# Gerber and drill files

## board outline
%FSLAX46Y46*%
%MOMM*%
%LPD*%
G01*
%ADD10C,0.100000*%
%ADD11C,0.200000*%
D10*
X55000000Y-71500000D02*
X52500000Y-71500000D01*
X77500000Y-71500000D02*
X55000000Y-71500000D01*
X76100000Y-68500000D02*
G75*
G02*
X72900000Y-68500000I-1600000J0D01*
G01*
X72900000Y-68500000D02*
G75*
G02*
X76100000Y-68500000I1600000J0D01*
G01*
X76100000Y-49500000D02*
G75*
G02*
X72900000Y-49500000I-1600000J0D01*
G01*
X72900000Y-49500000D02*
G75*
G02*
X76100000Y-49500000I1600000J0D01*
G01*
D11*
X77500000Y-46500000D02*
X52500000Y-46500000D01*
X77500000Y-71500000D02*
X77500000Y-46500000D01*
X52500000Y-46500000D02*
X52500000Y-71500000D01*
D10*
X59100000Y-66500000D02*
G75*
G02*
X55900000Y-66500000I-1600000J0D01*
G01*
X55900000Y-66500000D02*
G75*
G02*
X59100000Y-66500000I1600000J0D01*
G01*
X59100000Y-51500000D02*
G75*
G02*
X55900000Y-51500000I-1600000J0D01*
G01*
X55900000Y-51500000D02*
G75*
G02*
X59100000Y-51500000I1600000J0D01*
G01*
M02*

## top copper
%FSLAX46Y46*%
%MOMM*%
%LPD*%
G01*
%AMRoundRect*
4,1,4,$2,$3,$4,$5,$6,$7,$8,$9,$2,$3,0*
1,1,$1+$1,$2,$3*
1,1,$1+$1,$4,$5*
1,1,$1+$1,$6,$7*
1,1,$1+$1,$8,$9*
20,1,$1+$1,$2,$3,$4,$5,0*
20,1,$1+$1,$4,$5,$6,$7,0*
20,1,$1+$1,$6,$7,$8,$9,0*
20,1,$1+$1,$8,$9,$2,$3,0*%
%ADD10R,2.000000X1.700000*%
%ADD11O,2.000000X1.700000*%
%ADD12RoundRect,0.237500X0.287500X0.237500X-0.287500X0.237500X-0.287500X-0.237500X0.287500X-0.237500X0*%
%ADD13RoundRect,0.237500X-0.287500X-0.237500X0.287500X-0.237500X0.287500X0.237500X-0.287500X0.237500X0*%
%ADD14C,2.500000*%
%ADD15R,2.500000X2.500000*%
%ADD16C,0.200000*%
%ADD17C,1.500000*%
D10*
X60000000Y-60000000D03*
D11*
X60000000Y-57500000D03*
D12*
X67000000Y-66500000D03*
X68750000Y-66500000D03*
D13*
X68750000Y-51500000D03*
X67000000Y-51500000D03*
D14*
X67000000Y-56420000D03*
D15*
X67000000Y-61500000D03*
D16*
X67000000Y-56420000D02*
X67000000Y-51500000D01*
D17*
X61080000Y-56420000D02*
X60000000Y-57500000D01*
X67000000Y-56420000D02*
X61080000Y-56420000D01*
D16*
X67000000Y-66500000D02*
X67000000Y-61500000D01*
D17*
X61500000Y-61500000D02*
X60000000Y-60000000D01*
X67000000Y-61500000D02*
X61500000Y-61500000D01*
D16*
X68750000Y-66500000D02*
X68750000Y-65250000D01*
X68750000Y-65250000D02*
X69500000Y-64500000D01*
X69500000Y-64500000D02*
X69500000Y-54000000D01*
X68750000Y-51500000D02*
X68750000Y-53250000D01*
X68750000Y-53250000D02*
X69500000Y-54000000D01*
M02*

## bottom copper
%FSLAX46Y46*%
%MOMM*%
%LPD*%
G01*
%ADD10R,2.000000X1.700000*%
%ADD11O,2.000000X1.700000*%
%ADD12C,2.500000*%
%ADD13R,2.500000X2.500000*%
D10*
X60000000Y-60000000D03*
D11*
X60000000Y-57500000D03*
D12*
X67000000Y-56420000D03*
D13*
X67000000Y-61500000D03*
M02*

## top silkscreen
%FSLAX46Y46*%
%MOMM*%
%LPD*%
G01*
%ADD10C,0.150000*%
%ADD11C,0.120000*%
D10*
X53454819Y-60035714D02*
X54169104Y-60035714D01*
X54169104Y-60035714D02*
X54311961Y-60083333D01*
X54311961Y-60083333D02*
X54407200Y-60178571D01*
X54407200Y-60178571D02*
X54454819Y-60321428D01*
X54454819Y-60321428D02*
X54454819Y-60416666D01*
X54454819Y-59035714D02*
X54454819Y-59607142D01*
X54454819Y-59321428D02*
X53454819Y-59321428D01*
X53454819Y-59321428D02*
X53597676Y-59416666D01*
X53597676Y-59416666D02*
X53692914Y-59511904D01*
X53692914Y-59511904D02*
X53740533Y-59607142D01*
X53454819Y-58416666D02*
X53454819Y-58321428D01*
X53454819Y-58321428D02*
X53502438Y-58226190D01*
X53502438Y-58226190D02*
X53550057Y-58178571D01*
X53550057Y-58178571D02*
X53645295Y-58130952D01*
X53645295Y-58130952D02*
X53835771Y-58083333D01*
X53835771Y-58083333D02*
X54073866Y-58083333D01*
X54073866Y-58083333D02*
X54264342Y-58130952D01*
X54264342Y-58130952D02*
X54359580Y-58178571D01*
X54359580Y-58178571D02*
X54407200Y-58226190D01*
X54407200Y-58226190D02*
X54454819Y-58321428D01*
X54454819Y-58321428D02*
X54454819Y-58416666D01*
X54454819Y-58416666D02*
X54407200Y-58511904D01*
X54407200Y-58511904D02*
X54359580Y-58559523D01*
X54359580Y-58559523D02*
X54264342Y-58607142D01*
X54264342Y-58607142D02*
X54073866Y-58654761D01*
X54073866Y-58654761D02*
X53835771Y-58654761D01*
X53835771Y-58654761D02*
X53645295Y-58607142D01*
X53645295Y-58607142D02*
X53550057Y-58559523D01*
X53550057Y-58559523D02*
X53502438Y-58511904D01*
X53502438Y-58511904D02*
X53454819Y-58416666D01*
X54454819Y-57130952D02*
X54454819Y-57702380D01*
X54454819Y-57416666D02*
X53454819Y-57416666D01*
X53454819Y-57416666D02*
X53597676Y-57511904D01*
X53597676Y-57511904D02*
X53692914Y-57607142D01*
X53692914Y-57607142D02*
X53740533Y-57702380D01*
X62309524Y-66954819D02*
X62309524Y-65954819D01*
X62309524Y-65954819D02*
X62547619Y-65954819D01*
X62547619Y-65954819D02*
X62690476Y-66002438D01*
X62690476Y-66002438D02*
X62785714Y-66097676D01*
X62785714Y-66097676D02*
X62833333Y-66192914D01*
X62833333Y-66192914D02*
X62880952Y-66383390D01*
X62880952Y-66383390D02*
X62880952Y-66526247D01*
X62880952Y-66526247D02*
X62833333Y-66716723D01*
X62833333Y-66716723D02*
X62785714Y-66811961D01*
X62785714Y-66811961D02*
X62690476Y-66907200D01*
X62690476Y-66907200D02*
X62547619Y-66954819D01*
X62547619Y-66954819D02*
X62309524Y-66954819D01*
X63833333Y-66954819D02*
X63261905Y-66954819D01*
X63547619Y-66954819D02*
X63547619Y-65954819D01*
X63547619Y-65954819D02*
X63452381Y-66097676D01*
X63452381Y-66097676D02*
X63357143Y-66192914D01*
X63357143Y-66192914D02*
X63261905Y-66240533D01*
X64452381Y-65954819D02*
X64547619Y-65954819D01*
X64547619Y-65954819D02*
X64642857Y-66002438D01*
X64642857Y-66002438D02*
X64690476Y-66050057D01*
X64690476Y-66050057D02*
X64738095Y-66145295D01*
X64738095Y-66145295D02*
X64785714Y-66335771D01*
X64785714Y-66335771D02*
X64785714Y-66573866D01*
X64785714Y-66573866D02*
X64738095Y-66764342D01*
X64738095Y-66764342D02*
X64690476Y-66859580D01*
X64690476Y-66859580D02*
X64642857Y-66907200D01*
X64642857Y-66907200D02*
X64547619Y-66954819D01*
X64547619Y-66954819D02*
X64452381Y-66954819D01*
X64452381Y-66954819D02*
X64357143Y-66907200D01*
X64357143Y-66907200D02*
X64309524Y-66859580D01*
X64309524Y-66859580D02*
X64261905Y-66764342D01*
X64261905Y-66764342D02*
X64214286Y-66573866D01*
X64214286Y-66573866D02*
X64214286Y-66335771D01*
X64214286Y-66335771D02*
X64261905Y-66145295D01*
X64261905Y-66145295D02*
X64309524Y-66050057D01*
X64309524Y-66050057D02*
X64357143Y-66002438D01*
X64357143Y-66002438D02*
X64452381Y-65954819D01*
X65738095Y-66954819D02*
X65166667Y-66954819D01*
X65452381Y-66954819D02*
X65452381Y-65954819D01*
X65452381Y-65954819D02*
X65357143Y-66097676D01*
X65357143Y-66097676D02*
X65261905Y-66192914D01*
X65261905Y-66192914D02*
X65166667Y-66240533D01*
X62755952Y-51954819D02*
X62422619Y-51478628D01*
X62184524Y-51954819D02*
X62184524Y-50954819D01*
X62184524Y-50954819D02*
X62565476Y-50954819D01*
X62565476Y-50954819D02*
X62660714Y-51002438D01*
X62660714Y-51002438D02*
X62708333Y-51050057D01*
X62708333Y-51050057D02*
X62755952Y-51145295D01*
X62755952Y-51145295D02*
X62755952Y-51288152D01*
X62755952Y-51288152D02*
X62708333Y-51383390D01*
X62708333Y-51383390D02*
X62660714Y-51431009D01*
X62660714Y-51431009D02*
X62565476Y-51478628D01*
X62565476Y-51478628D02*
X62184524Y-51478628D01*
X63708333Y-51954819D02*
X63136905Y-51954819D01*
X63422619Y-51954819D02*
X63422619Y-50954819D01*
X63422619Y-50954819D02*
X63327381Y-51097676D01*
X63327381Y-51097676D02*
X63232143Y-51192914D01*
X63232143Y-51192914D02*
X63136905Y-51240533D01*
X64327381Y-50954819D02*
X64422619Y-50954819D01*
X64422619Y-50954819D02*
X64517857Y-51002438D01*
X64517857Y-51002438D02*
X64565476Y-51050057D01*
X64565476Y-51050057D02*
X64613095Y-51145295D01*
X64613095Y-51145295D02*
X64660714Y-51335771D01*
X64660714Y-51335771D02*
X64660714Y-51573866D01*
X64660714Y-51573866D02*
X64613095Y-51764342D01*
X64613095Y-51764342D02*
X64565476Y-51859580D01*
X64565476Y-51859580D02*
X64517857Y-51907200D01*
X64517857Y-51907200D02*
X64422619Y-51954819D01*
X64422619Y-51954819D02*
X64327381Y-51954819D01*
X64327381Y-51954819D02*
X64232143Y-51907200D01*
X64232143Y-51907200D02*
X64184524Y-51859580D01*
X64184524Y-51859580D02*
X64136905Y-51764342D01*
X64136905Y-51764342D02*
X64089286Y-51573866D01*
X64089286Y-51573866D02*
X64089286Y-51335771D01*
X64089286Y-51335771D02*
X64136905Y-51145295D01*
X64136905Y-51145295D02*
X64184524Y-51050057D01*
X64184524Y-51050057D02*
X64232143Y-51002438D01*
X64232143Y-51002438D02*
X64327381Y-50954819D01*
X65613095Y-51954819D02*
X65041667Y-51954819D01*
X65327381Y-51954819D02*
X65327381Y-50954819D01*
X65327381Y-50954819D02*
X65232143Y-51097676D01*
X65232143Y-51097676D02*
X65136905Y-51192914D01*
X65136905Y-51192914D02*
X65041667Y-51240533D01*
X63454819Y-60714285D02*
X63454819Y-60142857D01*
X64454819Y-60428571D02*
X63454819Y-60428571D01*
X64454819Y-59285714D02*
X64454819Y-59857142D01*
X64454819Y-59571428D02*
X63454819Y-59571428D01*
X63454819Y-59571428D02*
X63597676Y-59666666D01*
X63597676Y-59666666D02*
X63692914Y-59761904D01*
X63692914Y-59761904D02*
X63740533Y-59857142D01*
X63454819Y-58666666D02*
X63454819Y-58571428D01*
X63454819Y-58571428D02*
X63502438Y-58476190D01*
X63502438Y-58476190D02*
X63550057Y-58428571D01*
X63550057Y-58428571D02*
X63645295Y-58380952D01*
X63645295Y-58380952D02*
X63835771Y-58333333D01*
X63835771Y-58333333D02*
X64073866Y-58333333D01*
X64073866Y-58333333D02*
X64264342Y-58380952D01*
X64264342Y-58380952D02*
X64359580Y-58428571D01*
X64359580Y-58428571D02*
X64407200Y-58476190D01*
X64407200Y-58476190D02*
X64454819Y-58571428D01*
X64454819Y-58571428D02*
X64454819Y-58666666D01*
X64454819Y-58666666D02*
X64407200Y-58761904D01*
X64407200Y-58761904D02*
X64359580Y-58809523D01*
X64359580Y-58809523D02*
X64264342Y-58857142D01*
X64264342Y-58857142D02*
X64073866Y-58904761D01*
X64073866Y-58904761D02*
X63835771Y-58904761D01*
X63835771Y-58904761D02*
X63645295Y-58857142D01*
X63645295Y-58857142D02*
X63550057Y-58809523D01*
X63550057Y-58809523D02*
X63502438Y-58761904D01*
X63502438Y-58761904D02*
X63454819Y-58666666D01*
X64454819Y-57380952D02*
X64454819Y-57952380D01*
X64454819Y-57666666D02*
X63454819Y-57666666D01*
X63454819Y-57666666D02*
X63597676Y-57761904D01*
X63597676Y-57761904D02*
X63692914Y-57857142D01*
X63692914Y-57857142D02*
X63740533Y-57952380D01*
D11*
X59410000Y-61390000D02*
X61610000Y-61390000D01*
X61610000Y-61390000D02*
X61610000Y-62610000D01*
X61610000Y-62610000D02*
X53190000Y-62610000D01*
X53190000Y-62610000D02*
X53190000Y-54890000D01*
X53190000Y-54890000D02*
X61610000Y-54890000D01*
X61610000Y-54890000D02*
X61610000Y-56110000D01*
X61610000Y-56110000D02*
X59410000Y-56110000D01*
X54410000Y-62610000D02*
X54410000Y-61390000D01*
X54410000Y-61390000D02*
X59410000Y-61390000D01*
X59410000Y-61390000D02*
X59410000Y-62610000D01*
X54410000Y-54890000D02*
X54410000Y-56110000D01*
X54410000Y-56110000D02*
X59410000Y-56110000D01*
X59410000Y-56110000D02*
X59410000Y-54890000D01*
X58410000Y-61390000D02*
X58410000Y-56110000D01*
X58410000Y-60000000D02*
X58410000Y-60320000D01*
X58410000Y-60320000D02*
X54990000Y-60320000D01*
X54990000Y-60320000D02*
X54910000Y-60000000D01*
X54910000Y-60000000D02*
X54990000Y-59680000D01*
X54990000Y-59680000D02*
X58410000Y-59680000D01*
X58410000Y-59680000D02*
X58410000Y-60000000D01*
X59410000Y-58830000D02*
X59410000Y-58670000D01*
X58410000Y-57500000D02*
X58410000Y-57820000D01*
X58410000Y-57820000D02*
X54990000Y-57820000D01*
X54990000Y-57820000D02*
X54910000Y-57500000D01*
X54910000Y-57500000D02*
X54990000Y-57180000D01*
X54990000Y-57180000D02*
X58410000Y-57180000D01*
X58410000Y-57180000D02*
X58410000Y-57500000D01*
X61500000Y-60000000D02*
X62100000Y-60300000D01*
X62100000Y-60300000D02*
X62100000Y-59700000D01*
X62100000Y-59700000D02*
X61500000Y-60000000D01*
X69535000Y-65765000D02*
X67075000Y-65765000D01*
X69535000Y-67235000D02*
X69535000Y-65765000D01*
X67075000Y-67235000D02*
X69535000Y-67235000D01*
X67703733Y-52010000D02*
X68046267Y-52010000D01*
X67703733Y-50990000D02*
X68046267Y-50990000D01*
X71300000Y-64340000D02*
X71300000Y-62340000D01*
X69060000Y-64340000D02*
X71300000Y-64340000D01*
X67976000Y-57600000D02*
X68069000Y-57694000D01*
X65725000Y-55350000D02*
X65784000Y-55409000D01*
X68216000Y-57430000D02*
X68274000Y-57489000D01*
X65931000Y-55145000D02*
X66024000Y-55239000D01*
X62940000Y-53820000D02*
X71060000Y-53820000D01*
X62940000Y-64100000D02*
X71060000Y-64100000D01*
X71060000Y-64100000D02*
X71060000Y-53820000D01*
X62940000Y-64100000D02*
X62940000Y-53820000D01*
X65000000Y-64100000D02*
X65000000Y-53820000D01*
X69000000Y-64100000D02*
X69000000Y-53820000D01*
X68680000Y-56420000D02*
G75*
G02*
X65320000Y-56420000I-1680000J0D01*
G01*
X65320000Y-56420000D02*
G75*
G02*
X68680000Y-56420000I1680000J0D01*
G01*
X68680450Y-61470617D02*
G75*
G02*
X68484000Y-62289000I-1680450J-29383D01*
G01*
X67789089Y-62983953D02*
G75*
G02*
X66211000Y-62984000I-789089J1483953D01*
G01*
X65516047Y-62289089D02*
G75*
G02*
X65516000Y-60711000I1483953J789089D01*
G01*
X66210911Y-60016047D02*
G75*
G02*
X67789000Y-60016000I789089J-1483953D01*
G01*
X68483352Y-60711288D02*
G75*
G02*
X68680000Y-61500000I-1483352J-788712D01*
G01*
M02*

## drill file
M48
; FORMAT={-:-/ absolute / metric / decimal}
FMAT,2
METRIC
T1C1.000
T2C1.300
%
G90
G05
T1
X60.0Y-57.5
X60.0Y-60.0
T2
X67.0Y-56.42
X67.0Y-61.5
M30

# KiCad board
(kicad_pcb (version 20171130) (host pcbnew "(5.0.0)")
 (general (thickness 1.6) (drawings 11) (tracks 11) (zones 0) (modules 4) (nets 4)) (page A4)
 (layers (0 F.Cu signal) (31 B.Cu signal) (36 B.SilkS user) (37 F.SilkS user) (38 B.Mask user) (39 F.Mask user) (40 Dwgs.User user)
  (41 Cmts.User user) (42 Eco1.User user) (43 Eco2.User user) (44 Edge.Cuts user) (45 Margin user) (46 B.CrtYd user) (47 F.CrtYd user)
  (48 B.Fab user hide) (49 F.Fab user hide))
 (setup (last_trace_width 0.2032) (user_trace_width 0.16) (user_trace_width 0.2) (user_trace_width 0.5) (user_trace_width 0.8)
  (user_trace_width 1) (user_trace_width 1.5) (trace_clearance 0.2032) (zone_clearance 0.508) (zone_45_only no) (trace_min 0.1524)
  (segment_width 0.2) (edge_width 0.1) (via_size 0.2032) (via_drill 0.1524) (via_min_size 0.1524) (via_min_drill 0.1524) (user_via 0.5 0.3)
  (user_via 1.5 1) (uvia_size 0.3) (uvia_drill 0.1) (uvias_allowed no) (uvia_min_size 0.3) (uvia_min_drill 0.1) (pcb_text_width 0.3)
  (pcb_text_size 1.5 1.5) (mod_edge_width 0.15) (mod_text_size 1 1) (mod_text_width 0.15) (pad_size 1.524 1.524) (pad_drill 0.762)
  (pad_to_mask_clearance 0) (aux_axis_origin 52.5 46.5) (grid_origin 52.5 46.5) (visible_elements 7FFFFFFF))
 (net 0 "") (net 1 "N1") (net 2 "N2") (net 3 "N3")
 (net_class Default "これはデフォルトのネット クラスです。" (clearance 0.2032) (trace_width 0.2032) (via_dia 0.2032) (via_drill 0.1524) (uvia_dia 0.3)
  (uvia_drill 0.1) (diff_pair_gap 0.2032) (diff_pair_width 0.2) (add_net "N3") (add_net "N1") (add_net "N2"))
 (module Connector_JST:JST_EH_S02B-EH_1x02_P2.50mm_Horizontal (layer F.Cu) (at 60 60 90)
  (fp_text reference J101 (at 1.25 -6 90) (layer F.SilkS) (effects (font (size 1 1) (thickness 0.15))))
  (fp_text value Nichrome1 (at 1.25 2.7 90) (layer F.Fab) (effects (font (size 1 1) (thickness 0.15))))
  (fp_line (start -1.39 -0.59) (end -1.39 1.61) (layer F.SilkS) (width 0.12))
  (fp_line (start -1.39 1.61) (end -2.61 1.61) (layer F.SilkS) (width 0.12))
  (fp_line (start -2.61 1.61) (end -2.61 -6.81) (layer F.SilkS) (width 0.12))
  (fp_line (start -2.61 -6.81) (end 5.11 -6.81) (layer F.SilkS) (width 0.12))
  (fp_line (start 5.11 -6.81) (end 5.11 1.61) (layer F.SilkS) (width 0.12))
  (fp_line (start 5.11 1.61) (end 3.89 1.61) (layer F.SilkS) (width 0.12))
  (fp_line (start 3.89 1.61) (end 3.89 -0.59) (layer F.SilkS) (width 0.12))
  (fp_line (start -2.61 -5.59) (end -1.39 -5.59) (layer F.SilkS) (width 0.12))
  (fp_line (start -1.39 -5.59) (end -1.39 -0.59) (layer F.SilkS) (width 0.12))
  (fp_line (start -1.39 -0.59) (end -2.61 -0.59) (layer F.SilkS) (width 0.12))
  (fp_line (start 5.11 -5.59) (end 3.89 -5.59) (layer F.SilkS) (width 0.12))
  (fp_line (start 3.89 -5.59) (end 3.89 -0.59) (layer F.SilkS) (width 0.12))
  (fp_line (start 3.89 -0.59) (end 5.11 -0.59) (layer F.SilkS) (width 0.12))
  (fp_line (start -1.39 -1.59) (end 3.89 -1.59) (layer F.SilkS) (width 0.12))
  (fp_line (start 0 -1.59) (end -0.32 -1.59) (layer F.SilkS) (width 0.12))
  (fp_line (start -0.32 -1.59) (end -0.32 -5.01) (layer F.SilkS) (width 0.12))
  (fp_line (start -0.32 -5.01) (end 0 -5.09) (layer F.SilkS) (width 0.12))
  (fp_line (start 0 -5.09) (end 0.32 -5.01) (layer F.SilkS) (width 0.12))
  (fp_line (start 0.32 -5.01) (end 0.32 -1.59) (layer F.SilkS) (width 0.12))
  (fp_line (start 0.32 -1.59) (end 0 -1.59) (layer F.SilkS) (width 0.12))
  (fp_line (start 1.17 -0.59) (end 1.33 -0.59) (layer F.SilkS) (width 0.12))
  (fp_line (start 2.5 -1.59) (end 2.18 -1.59) (layer F.SilkS) (width 0.12))
  (fp_line (start 2.18 -1.59) (end 2.18 -5.01) (layer F.SilkS) (width 0.12))
  (fp_line (start 2.18 -5.01) (end 2.5 -5.09) (layer F.SilkS) (width 0.12))
  (fp_line (start 2.5 -5.09) (end 2.82 -5.01) (layer F.SilkS) (width 0.12))
  (fp_line (start 2.82 -5.01) (end 2.82 -1.59) (layer F.SilkS) (width 0.12))
  (fp_line (start 2.82 -1.59) (end 2.5 -1.59) (layer F.SilkS) (width 0.12))
  (fp_line (start 0 1.5) (end -0.3 2.1) (layer F.SilkS) (width 0.12))
  (fp_line (start -0.3 2.1) (end 0.3 2.1) (layer F.SilkS) (width 0.12))
  (fp_line (start 0.3 2.1) (end 0 1.5) (layer F.SilkS) (width 0.12))
  (pad 1 thru_hole rect (at 0 0 90) (size 1.7 2) (drill 1) (layers *.Cu *.Mask) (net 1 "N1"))
  (pad 2 thru_hole oval (at 2.5 0 90) (size 1.7 2) (drill 1) (layers *.Cu *.Mask) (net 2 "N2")))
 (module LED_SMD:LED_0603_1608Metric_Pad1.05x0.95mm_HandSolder (layer F.Cu) (at 67.875 66.5 180)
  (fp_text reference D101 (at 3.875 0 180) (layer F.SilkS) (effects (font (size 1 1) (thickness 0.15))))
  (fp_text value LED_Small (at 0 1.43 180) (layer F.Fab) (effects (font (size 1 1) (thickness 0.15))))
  (fp_line (start -1.66 0.735) (end 0.8 0.735) (layer F.SilkS) (width 0.12))
  (fp_line (start -1.66 -0.735) (end -1.66 0.735) (layer F.SilkS) (width 0.12))
  (fp_line (start 0.8 -0.735) (end -1.66 -0.735) (layer F.SilkS) (width 0.12))
  (pad 2 smd roundrect (at 0.875 0 180) (size 1.05 0.95) (layers F.Cu F.Paste F.Mask) (roundrect_rratio 0.25) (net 1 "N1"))
  (pad 1 smd roundrect (at -0.875 0 180) (size 1.05 0.95) (layers F.Cu F.Paste F.Mask) (roundrect_rratio 0.25) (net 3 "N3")))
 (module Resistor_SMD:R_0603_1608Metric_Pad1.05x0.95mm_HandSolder (layer F.Cu) (at 67.875 51.5)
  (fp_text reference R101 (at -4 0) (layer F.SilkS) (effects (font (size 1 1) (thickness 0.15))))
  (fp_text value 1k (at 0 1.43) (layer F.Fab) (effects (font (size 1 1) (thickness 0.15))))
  (fp_line (start -0.171267 0.51) (end 0.171267 0.51) (layer F.SilkS) (width 0.12))
  (fp_line (start -0.171267 -0.51) (end 0.171267 -0.51) (layer F.SilkS) (width 0.12))
  (pad 2 smd roundrect (at 0.875 0) (size 1.05 0.95) (layers F.Cu F.Paste F.Mask) (roundrect_rratio 0.25) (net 3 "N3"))
  (pad 1 smd roundrect (at -0.875 0) (size 1.05 0.95) (layers F.Cu F.Paste F.Mask) (roundrect_rratio 0.25) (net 2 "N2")))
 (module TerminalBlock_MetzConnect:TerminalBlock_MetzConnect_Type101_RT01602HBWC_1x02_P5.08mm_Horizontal (layer F.Cu) (at 67 61.5 90)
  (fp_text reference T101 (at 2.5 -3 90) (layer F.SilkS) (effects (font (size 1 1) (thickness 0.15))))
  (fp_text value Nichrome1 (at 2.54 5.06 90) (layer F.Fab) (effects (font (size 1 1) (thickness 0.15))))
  (fp_line (start -2.84 4.3) (end -0.84 4.3) (layer F.SilkS) (width 0.12))
  (fp_line (start -2.84 2.06) (end -2.84 4.3) (layer F.SilkS) (width 0.12))
  (fp_line (start 3.9 0.976) (end 3.806 1.069) (layer F.SilkS) (width 0.12))
  (fp_line (start 6.15 -1.275) (end 6.091 -1.216) (layer F.SilkS) (width 0.12))
  (fp_line (start 4.07 1.216) (end 4.011 1.274) (layer F.SilkS) (width 0.12))
  (fp_line (start 6.355 -1.069) (end 6.261 -0.976) (layer F.SilkS) (width 0.12))
  (fp_line (start 7.68 -4.06) (end 7.68 4.06) (layer F.SilkS) (width 0.12))
  (fp_line (start -2.6 -4.06) (end -2.6 4.06) (layer F.SilkS) (width 0.12))
  (fp_line (start -2.6 4.06) (end 7.68 4.06) (layer F.SilkS) (width 0.12))
  (fp_line (start -2.6 -4.06) (end 7.68 -4.06) (layer F.SilkS) (width 0.12))
  (fp_line (start -2.6 -2) (end 7.68 -2) (layer F.SilkS) (width 0.12))
  (fp_line (start -2.6 2) (end 7.68 2) (layer F.SilkS) (width 0.12))
  (fp_circle (center 5.08 0) (end 6.76 0) (layer F.SilkS) (width 0.12))
  (fp_arc (start 0 0) (end -0.789 1.484) (angle -29) (layer F.SilkS) (width 0.12))
  (fp_arc (start 0 0) (end -1.484 -0.789) (angle -56) (layer F.SilkS) (width 0.12))
  (fp_arc (start 0 0) (end 0.789 -1.484) (angle -56) (layer F.SilkS) (width 0.12))
  (fp_arc (start 0 0) (end 1.484 0.789) (angle -56) (layer F.SilkS) (width 0.12))
  (fp_arc (start 0 0) (end 0 1.68) (angle -28) (layer F.SilkS) (width 0.12))
  (pad 2 thru_hole circle (at 5.08 0 90) (size 2.5 2.5) (drill 1.3) (layers *.Cu *.Mask) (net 2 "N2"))
  (pad 1 thru_hole rect (at 0 0 90) (size 2.5 2.5) (drill 1.3) (layers *.Cu *.Mask) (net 1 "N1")))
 (gr_line (start 55 71.5) (end 52.5 71.5) (layer Edge.Cuts) (width 0.1))
 (gr_line (start 77.5 71.5) (end 55 71.5) (layer Edge.Cuts) (width 0.1))
 (gr_circle (center 74.5 68.5) (end 76.1 68.5) (layer Edge.Cuts) (width 0.1))
 (gr_circle (center 74.5 49.5) (end 76.1 49.5) (layer Edge.Cuts) (width 0.1))
 (gr_line (start 77.5 46.5) (end 52.5 46.5) (layer Edge.Cuts) (width 0.2))
 (gr_line (start 77.5 71.5) (end 77.5 46.5) (layer Edge.Cuts) (width 0.2))
 (gr_line (start 52.5 46.5) (end 52.5 71.5) (layer Edge.Cuts) (width 0.2))
 (gr_circle (center 57.5 66.5) (end 59.1 66.5) (layer Edge.Cuts) (width 0.1))
 (gr_circle (center 57.5 51.5) (end 59.1 51.5) (layer Edge.Cuts) (width 0.1))
 (segment (start 67 56.42) (end 67 51.5) (width 0.2) (layer F.Cu) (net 2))
 (segment (start 61.08 56.42) (end 60 57.5) (width 1.5) (layer F.Cu) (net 2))
 (segment (start 67 56.42) (end 61.08 56.42) (width 1.5) (layer F.Cu) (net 2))
 (segment (start 67 66.5) (end 67 61.5) (width 0.2) (layer F.Cu) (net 1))
 (segment (start 61.5 61.5) (end 60 60) (width 1.5) (layer F.Cu) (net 1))
 (segment (start 67 61.5) (end 61.5 61.5) (width 1.5) (layer F.Cu) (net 1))
 (segment (start 68.75 66.5) (end 68.75 65.25) (width 0.2) (layer F.Cu) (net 3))
 (segment (start 68.75 65.25) (end 69.5 64.5) (width 0.2) (layer F.Cu) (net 3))
 (segment (start 69.5 64.5) (end 69.5 54) (width 0.2) (layer F.Cu) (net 3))
 (segment (start 68.75 51.5) (end 68.75 53.25) (width 0.2) (layer F.Cu) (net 3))
 (segment (start 68.75 53.25) (end 69.5 54) (width 0.2) (layer F.Cu) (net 3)))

